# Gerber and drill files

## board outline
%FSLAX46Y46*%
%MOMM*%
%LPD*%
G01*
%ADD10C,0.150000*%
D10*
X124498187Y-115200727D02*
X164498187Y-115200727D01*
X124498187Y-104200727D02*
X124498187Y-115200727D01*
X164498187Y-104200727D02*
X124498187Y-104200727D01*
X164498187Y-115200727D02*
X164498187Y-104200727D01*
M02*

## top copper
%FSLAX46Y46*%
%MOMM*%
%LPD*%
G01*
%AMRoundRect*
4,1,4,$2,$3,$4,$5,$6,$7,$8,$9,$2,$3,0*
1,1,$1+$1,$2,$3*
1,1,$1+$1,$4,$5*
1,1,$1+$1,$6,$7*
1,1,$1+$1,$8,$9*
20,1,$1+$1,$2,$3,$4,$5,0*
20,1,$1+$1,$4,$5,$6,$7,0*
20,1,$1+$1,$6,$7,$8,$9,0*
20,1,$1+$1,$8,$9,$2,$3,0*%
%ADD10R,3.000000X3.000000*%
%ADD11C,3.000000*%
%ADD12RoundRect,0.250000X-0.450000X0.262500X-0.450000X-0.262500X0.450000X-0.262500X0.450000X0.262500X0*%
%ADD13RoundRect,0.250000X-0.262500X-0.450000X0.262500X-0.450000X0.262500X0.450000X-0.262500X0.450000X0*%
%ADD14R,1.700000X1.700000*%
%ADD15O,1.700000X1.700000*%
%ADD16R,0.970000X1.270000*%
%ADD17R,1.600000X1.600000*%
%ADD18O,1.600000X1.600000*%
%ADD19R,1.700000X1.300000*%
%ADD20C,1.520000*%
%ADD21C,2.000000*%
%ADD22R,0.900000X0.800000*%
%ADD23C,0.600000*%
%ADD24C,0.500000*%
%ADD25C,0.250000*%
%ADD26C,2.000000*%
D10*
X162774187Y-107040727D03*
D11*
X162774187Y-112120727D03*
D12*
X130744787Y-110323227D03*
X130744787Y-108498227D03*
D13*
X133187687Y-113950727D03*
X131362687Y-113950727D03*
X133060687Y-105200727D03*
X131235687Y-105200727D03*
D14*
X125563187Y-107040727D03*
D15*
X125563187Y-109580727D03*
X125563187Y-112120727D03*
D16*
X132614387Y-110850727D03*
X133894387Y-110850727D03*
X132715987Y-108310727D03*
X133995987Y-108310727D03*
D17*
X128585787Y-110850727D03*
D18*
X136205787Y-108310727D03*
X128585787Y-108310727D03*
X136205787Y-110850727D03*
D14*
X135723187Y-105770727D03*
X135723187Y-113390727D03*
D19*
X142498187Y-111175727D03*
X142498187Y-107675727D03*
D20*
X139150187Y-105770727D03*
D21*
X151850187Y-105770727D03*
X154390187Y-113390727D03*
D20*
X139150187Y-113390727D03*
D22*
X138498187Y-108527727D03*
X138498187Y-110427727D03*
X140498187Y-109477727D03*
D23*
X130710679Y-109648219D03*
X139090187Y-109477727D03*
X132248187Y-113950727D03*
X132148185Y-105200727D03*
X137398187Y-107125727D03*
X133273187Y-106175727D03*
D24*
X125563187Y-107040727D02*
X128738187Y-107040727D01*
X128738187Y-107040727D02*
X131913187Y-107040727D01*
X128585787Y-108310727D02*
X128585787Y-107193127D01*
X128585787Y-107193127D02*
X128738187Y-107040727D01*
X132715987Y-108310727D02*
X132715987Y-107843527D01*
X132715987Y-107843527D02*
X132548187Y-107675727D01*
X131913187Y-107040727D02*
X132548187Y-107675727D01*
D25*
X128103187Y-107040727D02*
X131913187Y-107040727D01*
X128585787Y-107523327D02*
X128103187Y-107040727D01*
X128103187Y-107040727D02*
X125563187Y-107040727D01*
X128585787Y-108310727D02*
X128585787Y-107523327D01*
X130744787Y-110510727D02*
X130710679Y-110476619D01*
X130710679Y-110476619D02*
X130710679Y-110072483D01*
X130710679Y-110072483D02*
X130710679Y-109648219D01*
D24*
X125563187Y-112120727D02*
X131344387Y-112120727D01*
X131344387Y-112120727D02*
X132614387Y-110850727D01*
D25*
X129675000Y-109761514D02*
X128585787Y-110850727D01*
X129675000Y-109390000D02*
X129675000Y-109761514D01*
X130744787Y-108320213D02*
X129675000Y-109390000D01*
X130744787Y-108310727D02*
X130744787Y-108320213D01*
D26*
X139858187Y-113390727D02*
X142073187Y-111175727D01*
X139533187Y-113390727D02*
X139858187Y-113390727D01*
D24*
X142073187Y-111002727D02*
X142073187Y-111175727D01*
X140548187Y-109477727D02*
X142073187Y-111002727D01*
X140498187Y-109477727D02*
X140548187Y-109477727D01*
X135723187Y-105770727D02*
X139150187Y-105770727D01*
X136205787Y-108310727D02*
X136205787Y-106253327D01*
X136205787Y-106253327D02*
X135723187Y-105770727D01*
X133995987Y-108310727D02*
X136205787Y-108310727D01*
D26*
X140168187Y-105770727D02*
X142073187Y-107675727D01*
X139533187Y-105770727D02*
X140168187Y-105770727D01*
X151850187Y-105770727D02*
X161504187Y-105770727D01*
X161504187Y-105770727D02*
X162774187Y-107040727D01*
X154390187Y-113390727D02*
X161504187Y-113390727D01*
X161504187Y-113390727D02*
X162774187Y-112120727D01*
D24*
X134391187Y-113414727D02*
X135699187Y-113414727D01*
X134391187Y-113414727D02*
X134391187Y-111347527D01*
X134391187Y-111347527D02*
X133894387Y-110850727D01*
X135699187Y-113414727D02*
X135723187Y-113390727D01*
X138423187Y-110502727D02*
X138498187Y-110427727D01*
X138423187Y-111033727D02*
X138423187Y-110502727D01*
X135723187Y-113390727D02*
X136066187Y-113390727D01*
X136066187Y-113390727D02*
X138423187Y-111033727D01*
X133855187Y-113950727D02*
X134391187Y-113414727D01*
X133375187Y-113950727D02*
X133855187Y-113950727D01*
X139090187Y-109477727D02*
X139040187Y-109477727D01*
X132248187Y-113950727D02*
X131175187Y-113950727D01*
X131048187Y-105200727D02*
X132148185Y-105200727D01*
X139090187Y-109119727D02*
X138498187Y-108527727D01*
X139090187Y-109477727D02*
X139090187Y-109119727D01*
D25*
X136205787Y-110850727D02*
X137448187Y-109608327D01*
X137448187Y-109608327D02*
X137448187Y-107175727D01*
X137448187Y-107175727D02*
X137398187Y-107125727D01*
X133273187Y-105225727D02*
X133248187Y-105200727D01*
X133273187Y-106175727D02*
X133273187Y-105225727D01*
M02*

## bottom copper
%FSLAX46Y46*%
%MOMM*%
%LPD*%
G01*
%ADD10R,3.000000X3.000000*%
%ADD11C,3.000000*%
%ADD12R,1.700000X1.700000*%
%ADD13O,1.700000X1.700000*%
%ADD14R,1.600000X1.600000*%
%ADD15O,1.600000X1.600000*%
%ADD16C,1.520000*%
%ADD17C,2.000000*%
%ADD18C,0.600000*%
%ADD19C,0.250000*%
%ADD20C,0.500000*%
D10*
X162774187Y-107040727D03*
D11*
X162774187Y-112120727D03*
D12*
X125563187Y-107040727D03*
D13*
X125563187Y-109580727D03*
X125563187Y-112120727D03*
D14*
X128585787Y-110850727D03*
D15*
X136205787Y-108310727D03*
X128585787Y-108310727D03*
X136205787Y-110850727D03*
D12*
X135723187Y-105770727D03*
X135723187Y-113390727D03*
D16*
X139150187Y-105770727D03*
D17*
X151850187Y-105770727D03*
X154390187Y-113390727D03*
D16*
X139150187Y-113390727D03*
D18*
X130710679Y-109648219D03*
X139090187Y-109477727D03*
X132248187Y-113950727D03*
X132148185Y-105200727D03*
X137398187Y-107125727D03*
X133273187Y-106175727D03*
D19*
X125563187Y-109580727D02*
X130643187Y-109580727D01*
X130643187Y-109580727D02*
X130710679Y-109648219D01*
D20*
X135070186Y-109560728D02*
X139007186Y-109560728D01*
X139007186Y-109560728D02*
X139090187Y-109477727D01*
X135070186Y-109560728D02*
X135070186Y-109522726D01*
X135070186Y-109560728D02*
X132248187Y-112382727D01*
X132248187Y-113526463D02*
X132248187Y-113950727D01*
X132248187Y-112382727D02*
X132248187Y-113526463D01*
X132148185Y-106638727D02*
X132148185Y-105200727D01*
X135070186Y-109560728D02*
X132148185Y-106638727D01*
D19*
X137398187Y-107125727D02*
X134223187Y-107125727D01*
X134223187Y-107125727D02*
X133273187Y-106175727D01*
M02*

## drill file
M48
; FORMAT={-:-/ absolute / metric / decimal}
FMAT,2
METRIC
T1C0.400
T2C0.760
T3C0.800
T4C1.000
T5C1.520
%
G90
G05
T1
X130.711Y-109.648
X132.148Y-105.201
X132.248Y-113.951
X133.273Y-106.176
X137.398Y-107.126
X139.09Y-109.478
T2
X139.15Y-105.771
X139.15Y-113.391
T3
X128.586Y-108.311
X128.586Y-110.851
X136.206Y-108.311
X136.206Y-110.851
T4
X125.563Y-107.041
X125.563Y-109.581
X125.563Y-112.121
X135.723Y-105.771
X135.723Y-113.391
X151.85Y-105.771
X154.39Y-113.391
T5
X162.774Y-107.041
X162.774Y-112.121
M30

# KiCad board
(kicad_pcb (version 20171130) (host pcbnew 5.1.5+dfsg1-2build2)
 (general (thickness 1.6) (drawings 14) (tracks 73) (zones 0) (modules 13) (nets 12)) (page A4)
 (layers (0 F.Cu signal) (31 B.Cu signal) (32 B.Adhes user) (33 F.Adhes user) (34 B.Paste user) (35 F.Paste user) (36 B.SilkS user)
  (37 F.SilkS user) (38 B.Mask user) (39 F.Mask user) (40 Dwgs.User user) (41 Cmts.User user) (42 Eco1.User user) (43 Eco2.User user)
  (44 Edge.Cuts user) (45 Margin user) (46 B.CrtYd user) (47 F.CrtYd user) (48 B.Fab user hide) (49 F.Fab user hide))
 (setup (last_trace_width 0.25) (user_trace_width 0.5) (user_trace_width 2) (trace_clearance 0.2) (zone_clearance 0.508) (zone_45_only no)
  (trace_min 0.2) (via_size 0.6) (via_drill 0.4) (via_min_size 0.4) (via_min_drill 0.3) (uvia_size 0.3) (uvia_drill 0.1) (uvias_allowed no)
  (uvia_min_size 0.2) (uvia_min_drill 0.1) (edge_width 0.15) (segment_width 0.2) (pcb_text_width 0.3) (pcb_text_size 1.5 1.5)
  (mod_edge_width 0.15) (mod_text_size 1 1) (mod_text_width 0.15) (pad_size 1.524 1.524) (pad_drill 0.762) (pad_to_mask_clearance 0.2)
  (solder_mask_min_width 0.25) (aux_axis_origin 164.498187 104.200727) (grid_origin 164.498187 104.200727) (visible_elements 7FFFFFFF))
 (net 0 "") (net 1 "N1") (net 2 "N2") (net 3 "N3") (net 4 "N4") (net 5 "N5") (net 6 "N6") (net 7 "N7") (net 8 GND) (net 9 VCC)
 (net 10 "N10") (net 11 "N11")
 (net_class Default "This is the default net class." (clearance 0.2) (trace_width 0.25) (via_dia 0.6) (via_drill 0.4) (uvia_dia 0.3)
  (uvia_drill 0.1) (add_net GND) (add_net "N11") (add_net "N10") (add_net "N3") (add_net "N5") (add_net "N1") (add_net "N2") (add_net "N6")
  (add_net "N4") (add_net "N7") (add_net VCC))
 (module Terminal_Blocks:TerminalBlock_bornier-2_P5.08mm (layer B.Cu) (at 162.774187 107.040727 270)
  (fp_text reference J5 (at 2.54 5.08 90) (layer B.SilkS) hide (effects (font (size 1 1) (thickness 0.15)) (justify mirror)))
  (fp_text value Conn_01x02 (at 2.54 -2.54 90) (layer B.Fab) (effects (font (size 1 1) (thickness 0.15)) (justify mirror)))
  (pad 1 thru_hole rect (at 0 0 270) (size 3 3) (drill 1.52) (layers *.Cu *.Mask) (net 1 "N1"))
  (pad 2 thru_hole circle (at 5.08 0 270) (size 3 3) (drill 1.52) (layers *.Cu *.Mask) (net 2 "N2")))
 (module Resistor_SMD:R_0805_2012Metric (layer F.Cu) (at 130.744787 109.410727 270)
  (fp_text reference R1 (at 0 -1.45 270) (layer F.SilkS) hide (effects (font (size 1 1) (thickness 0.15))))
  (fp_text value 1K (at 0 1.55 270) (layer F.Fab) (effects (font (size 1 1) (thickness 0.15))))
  (pad 2 smd roundrect (at 0.9125 0 270) (size 1.025 1.4) (layers F.Cu F.Paste F.Mask) (roundrect_rratio 0.243902) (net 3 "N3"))
  (pad 1 smd roundrect (at -0.9125 0 270) (size 1.025 1.4) (layers F.Cu F.Paste F.Mask) (roundrect_rratio 0.243902) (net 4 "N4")))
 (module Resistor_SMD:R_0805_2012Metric (layer F.Cu) (at 132.275187 113.950727)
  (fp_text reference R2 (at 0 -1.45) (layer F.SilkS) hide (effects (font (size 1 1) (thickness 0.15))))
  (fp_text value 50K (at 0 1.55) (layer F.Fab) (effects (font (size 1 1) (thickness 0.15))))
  (pad 2 smd roundrect (at 0.9125 0) (size 1.025 1.4) (layers F.Cu F.Paste F.Mask) (roundrect_rratio 0.243902) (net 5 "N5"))
  (pad 1 smd roundrect (at -0.9125 0) (size 1.025 1.4) (layers F.Cu F.Paste F.Mask) (roundrect_rratio 0.243902) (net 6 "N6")))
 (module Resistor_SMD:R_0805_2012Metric (layer F.Cu) (at 132.148187 105.200727)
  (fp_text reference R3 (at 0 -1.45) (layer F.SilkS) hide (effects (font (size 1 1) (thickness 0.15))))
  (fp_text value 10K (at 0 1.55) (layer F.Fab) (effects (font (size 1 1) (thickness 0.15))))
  (pad 2 smd roundrect (at 0.9125 0) (size 1.025 1.4) (layers F.Cu F.Paste F.Mask) (roundrect_rratio 0.243902) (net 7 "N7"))
  (pad 1 smd roundrect (at -0.9125 0) (size 1.025 1.4) (layers F.Cu F.Paste F.Mask) (roundrect_rratio 0.243902) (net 6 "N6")))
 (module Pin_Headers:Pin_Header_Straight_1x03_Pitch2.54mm (layer B.Cu) (at 125.563187 107.040727 180)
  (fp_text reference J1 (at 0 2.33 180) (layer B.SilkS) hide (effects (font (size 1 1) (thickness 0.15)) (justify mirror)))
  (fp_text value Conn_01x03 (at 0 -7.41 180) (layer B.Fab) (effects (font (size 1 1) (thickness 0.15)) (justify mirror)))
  (pad 1 thru_hole rect (at 0 0 180) (size 1.7 1.7) (drill 1) (layers *.Cu *.Mask) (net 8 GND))
  (pad 2 thru_hole oval (at 0 -2.54 180) (size 1.7 1.7) (drill 1) (layers *.Cu *.Mask) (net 3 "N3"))
  (pad 3 thru_hole oval (at 0 -5.08 180) (size 1.7 1.7) (drill 1) (layers *.Cu *.Mask) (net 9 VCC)))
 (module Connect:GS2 (layer F.Cu) (at 133.254387 110.850727 90)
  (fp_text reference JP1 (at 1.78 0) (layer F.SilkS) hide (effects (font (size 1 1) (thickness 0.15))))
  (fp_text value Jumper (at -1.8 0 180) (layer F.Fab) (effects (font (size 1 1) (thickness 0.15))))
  (pad 1 smd rect (at 0 -0.64 90) (size 1.27 0.97) (layers F.Cu F.Paste F.Mask) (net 9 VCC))
  (pad 2 smd rect (at 0 0.64 90) (size 1.27 0.97) (layers F.Cu F.Paste F.Mask) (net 5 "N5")))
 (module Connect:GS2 (layer F.Cu) (at 133.355987 108.310727 90)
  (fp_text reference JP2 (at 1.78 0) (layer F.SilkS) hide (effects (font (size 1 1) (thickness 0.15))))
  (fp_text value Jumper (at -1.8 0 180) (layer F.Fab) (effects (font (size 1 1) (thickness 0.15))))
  (pad 1 smd rect (at 0 -0.64 90) (size 1.27 0.97) (layers F.Cu F.Paste F.Mask) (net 8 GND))
  (pad 2 smd rect (at 0 0.64 90) (size 1.27 0.97) (layers F.Cu F.Paste F.Mask) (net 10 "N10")))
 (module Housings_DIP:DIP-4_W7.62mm (layer B.Cu) (at 128.585787 110.850727)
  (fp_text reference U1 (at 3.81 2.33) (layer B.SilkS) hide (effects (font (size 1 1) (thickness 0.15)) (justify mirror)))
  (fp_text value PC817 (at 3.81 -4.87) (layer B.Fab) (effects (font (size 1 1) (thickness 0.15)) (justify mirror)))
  (pad 1 thru_hole rect (at 0 0) (size 1.6 1.6) (drill 0.8) (layers *.Cu *.Mask) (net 4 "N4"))
  (pad 3 thru_hole oval (at 7.62 -2.54) (size 1.6 1.6) (drill 0.8) (layers *.Cu *.Mask) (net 10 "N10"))
  (pad 2 thru_hole oval (at 0 -2.54) (size 1.6 1.6) (drill 0.8) (layers *.Cu *.Mask) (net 8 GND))
  (pad 4 thru_hole oval (at 7.62 0) (size 1.6 1.6) (drill 0.8) (layers *.Cu *.Mask) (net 7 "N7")))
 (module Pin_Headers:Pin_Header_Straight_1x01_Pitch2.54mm (layer B.Cu) (at 135.723187 105.770727 270)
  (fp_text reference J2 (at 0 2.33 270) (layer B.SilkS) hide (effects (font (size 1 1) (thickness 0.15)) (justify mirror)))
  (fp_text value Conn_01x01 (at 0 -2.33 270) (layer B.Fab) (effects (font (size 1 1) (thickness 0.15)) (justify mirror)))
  (pad 1 thru_hole rect (at 0 0 270) (size 1.7 1.7) (drill 1) (layers *.Cu *.Mask) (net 10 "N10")))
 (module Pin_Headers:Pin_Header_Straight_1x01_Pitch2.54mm (layer B.Cu) (at 135.723187 113.390727)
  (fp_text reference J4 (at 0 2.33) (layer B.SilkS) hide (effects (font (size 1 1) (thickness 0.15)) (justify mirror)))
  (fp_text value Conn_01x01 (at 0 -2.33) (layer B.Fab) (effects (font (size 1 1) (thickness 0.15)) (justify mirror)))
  (pad 1 thru_hole rect (at 0 0) (size 1.7 1.7) (drill 1) (layers *.Cu *.Mask) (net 5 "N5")))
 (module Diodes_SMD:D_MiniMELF (layer F.Cu) (at 142.498187 109.425727 90)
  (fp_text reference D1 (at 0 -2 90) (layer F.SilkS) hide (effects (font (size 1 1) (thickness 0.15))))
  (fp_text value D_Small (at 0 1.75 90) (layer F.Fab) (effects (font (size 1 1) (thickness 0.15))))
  (pad 1 smd rect (at -1.75 0 90) (size 1.3 1.7) (layers F.Cu F.Paste F.Mask) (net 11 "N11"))
  (pad 2 smd rect (at 1.75 0 90) (size 1.3 1.7) (layers F.Cu F.Paste F.Mask) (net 10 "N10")))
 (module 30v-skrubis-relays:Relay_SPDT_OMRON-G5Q (layer B.Cu) (at 139.150187 105.770727)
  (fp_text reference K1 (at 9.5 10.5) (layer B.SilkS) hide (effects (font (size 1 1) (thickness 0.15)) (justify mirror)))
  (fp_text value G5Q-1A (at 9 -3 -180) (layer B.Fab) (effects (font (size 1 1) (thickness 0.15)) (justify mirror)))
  (pad 1 thru_hole circle (at 0 0 180) (size 1.52 1.52) (drill 0.76) (layers *.Cu *.Mask) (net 10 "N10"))
  (pad 2 thru_hole circle (at 12.7 0 180) (size 2 2) (drill 1) (layers *.Cu *.Mask) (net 1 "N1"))
  (pad 3 thru_hole circle (at 15.24 7.62 180) (size 2 2) (drill 1) (layers *.Cu *.Mask) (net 2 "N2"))
  (pad 5 thru_hole circle (at 0 7.62 180) (size 1.52 1.52) (drill 0.76) (layers *.Cu *.Mask) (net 11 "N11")))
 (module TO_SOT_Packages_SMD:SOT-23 (layer F.Cu) (at 139.498187 109.477727)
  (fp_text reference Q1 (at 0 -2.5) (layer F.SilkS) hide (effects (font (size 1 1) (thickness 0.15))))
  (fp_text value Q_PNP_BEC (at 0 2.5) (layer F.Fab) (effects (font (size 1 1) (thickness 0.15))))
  (pad 1 smd rect (at -1 -0.95) (size 0.9 0.8) (layers F.Cu F.Paste F.Mask) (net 6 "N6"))
  (pad 2 smd rect (at -1 0.95) (size 0.9 0.8) (layers F.Cu F.Paste F.Mask) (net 5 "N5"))
  (pad 3 smd rect (at 1 0) (size 0.9 0.8) (layers F.Cu F.Paste F.Mask) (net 11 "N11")))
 (gr_line (start 124.498187 115.200727) (end 164.498187 115.200727) (layer Edge.Cuts) (width 0.15))
 (gr_line (start 124.498187 104.200727) (end 124.498187 115.200727) (layer Edge.Cuts) (width 0.15))
 (gr_line (start 164.498187 104.200727) (end 124.498187 104.200727) (layer Edge.Cuts) (width 0.15))
 (gr_line (start 164.498187 115.200727) (end 164.498187 104.200727) (layer Edge.Cuts) (width 0.15))
 (segment (start 125.563187 107.040727) (end 128.738187 107.040727) (width 0.5) (layer F.Cu) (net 8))
 (segment (start 128.738187 107.040727) (end 131.913187 107.040727) (width 0.5) (layer F.Cu) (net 8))
 (segment (start 128.585787 108.310727) (end 128.585787 107.193127) (width 0.5) (layer F.Cu) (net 8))
 (segment (start 128.585787 107.193127) (end 128.738187 107.040727) (width 0.5) (layer F.Cu) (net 8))
 (segment (start 132.715987 108.310727) (end 132.715987 107.843527) (width 0.5) (layer F.Cu) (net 8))
 (segment (start 132.715987 107.843527) (end 132.548187 107.675727) (width 0.5) (layer F.Cu) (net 8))
 (segment (start 131.913187 107.040727) (end 132.548187 107.675727) (width 0.5) (layer F.Cu) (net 8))
 (segment (start 128.103187 107.040727) (end 131.913187 107.040727) (width 0.25) (layer F.Cu) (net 8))
 (segment (start 128.585787 107.523327) (end 128.103187 107.040727) (width 0.25) (layer F.Cu) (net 8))
 (segment (start 128.103187 107.040727) (end 125.563187 107.040727) (width 0.25) (layer F.Cu) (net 8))
 (segment (start 128.585787 108.310727) (end 128.585787 107.523327) (width 0.25) (layer F.Cu) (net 8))
 (segment (start 130.744787 110.510727) (end 130.710679 110.476619) (width 0.25) (layer F.Cu) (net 3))
 (segment (start 125.563187 109.580727) (end 130.643187 109.580727) (width 0.25) (layer B.Cu) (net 3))
 (via (at 130.710679 109.648219) (size 0.6) (drill 0.4) (layers F.Cu B.Cu) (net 3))
 (segment (start 130.643187 109.580727) (end 130.710679 109.648219) (width 0.25) (layer B.Cu) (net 3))
 (segment (start 130.710679 110.476619) (end 130.710679 110.072483) (width 0.25) (layer F.Cu) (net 3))
 (segment (start 130.710679 110.072483) (end 130.710679 109.648219) (width 0.25) (layer F.Cu) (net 3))
 (segment (start 125.563187 112.120727) (end 131.344387 112.120727) (width 0.5) (layer F.Cu) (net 9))
 (segment (start 131.344387 112.120727) (end 132.614387 110.850727) (width 0.5) (layer F.Cu) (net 9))
 (segment (start 129.675 109.761514) (end 128.585787 110.850727) (width 0.25) (layer F.Cu) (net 4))
 (segment (start 129.675 109.39) (end 129.675 109.761514) (width 0.25) (layer F.Cu) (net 4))
 (segment (start 130.744787 108.320213) (end 129.675 109.39) (width 0.25) (layer F.Cu) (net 4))
 (segment (start 130.744787 108.310727) (end 130.744787 108.320213) (width 0.25) (layer F.Cu) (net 4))
 (segment (start 139.858187 113.390727) (end 142.073187 111.175727) (width 2) (layer F.Cu) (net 11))
 (segment (start 139.533187 113.390727) (end 139.858187 113.390727) (width 2) (layer F.Cu) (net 11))
 (segment (start 142.073187 111.002727) (end 142.073187 111.175727) (width 0.5) (layer F.Cu) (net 11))
 (segment (start 140.548187 109.477727) (end 142.073187 111.002727) (width 0.5) (layer F.Cu) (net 11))
 (segment (start 140.498187 109.477727) (end 140.548187 109.477727) (width 0.5) (layer F.Cu) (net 11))
 (segment (start 135.723187 105.770727) (end 139.150187 105.770727) (width 0.5) (layer F.Cu) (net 10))
 (segment (start 136.205787 108.310727) (end 136.205787 106.253327) (width 0.5) (layer F.Cu) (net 10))
 (segment (start 136.205787 106.253327) (end 135.723187 105.770727) (width 0.5) (layer F.Cu) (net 10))
 (segment (start 133.995987 108.310727) (end 136.205787 108.310727) (width 0.5) (layer F.Cu) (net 10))
 (segment (start 140.168187 105.770727) (end 142.073187 107.675727) (width 2) (layer F.Cu) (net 10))
 (segment (start 139.533187 105.770727) (end 140.168187 105.770727) (width 2) (layer F.Cu) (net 10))
 (segment (start 151.850187 105.770727) (end 161.504187 105.770727) (width 2) (layer F.Cu) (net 1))
 (segment (start 161.504187 105.770727) (end 162.774187 107.040727) (width 2) (layer F.Cu) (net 1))
 (segment (start 154.390187 113.390727) (end 161.504187 113.390727) (width 2) (layer F.Cu) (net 2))
 (segment (start 161.504187 113.390727) (end 162.774187 112.120727) (width 2) (layer F.Cu) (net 2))
 (segment (start 134.391187 113.414727) (end 135.699187 113.414727) (width 0.5) (layer F.Cu) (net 5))
 (segment (start 134.391187 113.414727) (end 134.391187 111.347527) (width 0.5) (layer F.Cu) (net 5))
 (segment (start 134.391187 111.347527) (end 133.894387 110.850727) (width 0.5) (layer F.Cu) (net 5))
 (segment (start 135.699187 113.414727) (end 135.723187 113.390727) (width 0.5) (layer F.Cu) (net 5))
 (segment (start 138.423187 110.502727) (end 138.498187 110.427727) (width 0.5) (layer F.Cu) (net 5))
 (segment (start 138.423187 111.033727) (end 138.423187 110.502727) (width 0.5) (layer F.Cu) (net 5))
 (segment (start 135.723187 113.390727) (end 136.066187 113.390727) (width 0.5) (layer F.Cu) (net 5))
 (segment (start 136.066187 113.390727) (end 138.423187 111.033727) (width 0.5) (layer F.Cu) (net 5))
 (segment (start 133.855187 113.950727) (end 134.391187 113.414727) (width 0.5) (layer F.Cu) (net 5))
 (segment (start 133.375187 113.950727) (end 133.855187 113.950727) (width 0.5) (layer F.Cu) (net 5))
 (segment (start 139.090187 109.477727) (end 139.040187 109.477727) (width 0.5) (layer F.Cu) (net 6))
 (segment (start 135.070186 109.560728) (end 139.007186 109.560728) (width 0.5) (layer B.Cu) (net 6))
 (segment (start 139.007186 109.560728) (end 139.090187 109.477727) (width 0.5) (layer B.Cu) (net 6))
 (via (at 139.090187 109.477727) (size 0.6) (drill 0.4) (layers F.Cu B.Cu) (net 6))
 (segment (start 135.070186 109.560728) (end 135.070186 109.522726) (width 0.5) (layer B.Cu) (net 6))
 (segment (start 135.070186 109.560728) (end 132.248187 112.382727) (width 0.5) (layer B.Cu) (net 6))
 (via (at 132.248187 113.950727) (size 0.6) (drill 0.4) (layers F.Cu B.Cu) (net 6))
 (segment (start 132.248187 113.526463) (end 132.248187 113.950727) (width 0.5) (layer B.Cu) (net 6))
 (segment (start 132.248187 112.382727) (end 132.248187 113.526463) (width 0.5) (layer B.Cu) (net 6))
 (segment (start 132.248187 113.950727) (end 131.175187 113.950727) (width 0.5) (layer F.Cu) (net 6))
 (via (at 132.148185 105.200727) (size 0.6) (drill 0.4) (layers F.Cu B.Cu) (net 6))
 (segment (start 131.048187 105.200727) (end 132.148185 105.200727) (width 0.5) (layer F.Cu) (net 6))
 (segment (start 132.148185 106.638727) (end 132.148185 105.200727) (width 0.5) (layer B.Cu) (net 6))
 (segment (start 135.070186 109.560728) (end 132.148185 106.638727) (width 0.5) (layer B.Cu) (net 6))
 (segment (start 139.090187 109.119727) (end 138.498187 108.527727) (width 0.5) (layer F.Cu) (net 6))
 (segment (start 139.090187 109.477727) (end 139.090187 109.119727) (width 0.5) (layer F.Cu) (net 6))
 (segment (start 136.205787 110.850727) (end 137.448187 109.608327) (width 0.25) (layer F.Cu) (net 7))
 (via (at 137.398187 107.125727) (size 0.6) (drill 0.4) (layers F.Cu B.Cu) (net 7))
 (segment (start 137.448187 109.608327) (end 137.448187 107.175727) (width 0.25) (layer F.Cu) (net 7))
 (segment (start 137.448187 107.175727) (end 137.398187 107.125727) (width 0.25) (layer F.Cu) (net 7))
 (via (at 133.273187 106.175727) (size 0.6) (drill 0.4) (layers F.Cu B.Cu) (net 7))
 (segment (start 137.398187 107.125727) (end 134.223187 107.125727) (width 0.25) (layer B.Cu) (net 7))
 (segment (start 134.223187 107.125727) (end 133.273187 106.175727) (width 0.25) (layer B.Cu) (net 7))
 (segment (start 133.273187 105.225727) (end 133.248187 105.200727) (width 0.25) (layer F.Cu) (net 7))
 (segment (start 133.273187 106.175727) (end 133.273187 105.225727) (width 0.25) (layer F.Cu) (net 7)))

